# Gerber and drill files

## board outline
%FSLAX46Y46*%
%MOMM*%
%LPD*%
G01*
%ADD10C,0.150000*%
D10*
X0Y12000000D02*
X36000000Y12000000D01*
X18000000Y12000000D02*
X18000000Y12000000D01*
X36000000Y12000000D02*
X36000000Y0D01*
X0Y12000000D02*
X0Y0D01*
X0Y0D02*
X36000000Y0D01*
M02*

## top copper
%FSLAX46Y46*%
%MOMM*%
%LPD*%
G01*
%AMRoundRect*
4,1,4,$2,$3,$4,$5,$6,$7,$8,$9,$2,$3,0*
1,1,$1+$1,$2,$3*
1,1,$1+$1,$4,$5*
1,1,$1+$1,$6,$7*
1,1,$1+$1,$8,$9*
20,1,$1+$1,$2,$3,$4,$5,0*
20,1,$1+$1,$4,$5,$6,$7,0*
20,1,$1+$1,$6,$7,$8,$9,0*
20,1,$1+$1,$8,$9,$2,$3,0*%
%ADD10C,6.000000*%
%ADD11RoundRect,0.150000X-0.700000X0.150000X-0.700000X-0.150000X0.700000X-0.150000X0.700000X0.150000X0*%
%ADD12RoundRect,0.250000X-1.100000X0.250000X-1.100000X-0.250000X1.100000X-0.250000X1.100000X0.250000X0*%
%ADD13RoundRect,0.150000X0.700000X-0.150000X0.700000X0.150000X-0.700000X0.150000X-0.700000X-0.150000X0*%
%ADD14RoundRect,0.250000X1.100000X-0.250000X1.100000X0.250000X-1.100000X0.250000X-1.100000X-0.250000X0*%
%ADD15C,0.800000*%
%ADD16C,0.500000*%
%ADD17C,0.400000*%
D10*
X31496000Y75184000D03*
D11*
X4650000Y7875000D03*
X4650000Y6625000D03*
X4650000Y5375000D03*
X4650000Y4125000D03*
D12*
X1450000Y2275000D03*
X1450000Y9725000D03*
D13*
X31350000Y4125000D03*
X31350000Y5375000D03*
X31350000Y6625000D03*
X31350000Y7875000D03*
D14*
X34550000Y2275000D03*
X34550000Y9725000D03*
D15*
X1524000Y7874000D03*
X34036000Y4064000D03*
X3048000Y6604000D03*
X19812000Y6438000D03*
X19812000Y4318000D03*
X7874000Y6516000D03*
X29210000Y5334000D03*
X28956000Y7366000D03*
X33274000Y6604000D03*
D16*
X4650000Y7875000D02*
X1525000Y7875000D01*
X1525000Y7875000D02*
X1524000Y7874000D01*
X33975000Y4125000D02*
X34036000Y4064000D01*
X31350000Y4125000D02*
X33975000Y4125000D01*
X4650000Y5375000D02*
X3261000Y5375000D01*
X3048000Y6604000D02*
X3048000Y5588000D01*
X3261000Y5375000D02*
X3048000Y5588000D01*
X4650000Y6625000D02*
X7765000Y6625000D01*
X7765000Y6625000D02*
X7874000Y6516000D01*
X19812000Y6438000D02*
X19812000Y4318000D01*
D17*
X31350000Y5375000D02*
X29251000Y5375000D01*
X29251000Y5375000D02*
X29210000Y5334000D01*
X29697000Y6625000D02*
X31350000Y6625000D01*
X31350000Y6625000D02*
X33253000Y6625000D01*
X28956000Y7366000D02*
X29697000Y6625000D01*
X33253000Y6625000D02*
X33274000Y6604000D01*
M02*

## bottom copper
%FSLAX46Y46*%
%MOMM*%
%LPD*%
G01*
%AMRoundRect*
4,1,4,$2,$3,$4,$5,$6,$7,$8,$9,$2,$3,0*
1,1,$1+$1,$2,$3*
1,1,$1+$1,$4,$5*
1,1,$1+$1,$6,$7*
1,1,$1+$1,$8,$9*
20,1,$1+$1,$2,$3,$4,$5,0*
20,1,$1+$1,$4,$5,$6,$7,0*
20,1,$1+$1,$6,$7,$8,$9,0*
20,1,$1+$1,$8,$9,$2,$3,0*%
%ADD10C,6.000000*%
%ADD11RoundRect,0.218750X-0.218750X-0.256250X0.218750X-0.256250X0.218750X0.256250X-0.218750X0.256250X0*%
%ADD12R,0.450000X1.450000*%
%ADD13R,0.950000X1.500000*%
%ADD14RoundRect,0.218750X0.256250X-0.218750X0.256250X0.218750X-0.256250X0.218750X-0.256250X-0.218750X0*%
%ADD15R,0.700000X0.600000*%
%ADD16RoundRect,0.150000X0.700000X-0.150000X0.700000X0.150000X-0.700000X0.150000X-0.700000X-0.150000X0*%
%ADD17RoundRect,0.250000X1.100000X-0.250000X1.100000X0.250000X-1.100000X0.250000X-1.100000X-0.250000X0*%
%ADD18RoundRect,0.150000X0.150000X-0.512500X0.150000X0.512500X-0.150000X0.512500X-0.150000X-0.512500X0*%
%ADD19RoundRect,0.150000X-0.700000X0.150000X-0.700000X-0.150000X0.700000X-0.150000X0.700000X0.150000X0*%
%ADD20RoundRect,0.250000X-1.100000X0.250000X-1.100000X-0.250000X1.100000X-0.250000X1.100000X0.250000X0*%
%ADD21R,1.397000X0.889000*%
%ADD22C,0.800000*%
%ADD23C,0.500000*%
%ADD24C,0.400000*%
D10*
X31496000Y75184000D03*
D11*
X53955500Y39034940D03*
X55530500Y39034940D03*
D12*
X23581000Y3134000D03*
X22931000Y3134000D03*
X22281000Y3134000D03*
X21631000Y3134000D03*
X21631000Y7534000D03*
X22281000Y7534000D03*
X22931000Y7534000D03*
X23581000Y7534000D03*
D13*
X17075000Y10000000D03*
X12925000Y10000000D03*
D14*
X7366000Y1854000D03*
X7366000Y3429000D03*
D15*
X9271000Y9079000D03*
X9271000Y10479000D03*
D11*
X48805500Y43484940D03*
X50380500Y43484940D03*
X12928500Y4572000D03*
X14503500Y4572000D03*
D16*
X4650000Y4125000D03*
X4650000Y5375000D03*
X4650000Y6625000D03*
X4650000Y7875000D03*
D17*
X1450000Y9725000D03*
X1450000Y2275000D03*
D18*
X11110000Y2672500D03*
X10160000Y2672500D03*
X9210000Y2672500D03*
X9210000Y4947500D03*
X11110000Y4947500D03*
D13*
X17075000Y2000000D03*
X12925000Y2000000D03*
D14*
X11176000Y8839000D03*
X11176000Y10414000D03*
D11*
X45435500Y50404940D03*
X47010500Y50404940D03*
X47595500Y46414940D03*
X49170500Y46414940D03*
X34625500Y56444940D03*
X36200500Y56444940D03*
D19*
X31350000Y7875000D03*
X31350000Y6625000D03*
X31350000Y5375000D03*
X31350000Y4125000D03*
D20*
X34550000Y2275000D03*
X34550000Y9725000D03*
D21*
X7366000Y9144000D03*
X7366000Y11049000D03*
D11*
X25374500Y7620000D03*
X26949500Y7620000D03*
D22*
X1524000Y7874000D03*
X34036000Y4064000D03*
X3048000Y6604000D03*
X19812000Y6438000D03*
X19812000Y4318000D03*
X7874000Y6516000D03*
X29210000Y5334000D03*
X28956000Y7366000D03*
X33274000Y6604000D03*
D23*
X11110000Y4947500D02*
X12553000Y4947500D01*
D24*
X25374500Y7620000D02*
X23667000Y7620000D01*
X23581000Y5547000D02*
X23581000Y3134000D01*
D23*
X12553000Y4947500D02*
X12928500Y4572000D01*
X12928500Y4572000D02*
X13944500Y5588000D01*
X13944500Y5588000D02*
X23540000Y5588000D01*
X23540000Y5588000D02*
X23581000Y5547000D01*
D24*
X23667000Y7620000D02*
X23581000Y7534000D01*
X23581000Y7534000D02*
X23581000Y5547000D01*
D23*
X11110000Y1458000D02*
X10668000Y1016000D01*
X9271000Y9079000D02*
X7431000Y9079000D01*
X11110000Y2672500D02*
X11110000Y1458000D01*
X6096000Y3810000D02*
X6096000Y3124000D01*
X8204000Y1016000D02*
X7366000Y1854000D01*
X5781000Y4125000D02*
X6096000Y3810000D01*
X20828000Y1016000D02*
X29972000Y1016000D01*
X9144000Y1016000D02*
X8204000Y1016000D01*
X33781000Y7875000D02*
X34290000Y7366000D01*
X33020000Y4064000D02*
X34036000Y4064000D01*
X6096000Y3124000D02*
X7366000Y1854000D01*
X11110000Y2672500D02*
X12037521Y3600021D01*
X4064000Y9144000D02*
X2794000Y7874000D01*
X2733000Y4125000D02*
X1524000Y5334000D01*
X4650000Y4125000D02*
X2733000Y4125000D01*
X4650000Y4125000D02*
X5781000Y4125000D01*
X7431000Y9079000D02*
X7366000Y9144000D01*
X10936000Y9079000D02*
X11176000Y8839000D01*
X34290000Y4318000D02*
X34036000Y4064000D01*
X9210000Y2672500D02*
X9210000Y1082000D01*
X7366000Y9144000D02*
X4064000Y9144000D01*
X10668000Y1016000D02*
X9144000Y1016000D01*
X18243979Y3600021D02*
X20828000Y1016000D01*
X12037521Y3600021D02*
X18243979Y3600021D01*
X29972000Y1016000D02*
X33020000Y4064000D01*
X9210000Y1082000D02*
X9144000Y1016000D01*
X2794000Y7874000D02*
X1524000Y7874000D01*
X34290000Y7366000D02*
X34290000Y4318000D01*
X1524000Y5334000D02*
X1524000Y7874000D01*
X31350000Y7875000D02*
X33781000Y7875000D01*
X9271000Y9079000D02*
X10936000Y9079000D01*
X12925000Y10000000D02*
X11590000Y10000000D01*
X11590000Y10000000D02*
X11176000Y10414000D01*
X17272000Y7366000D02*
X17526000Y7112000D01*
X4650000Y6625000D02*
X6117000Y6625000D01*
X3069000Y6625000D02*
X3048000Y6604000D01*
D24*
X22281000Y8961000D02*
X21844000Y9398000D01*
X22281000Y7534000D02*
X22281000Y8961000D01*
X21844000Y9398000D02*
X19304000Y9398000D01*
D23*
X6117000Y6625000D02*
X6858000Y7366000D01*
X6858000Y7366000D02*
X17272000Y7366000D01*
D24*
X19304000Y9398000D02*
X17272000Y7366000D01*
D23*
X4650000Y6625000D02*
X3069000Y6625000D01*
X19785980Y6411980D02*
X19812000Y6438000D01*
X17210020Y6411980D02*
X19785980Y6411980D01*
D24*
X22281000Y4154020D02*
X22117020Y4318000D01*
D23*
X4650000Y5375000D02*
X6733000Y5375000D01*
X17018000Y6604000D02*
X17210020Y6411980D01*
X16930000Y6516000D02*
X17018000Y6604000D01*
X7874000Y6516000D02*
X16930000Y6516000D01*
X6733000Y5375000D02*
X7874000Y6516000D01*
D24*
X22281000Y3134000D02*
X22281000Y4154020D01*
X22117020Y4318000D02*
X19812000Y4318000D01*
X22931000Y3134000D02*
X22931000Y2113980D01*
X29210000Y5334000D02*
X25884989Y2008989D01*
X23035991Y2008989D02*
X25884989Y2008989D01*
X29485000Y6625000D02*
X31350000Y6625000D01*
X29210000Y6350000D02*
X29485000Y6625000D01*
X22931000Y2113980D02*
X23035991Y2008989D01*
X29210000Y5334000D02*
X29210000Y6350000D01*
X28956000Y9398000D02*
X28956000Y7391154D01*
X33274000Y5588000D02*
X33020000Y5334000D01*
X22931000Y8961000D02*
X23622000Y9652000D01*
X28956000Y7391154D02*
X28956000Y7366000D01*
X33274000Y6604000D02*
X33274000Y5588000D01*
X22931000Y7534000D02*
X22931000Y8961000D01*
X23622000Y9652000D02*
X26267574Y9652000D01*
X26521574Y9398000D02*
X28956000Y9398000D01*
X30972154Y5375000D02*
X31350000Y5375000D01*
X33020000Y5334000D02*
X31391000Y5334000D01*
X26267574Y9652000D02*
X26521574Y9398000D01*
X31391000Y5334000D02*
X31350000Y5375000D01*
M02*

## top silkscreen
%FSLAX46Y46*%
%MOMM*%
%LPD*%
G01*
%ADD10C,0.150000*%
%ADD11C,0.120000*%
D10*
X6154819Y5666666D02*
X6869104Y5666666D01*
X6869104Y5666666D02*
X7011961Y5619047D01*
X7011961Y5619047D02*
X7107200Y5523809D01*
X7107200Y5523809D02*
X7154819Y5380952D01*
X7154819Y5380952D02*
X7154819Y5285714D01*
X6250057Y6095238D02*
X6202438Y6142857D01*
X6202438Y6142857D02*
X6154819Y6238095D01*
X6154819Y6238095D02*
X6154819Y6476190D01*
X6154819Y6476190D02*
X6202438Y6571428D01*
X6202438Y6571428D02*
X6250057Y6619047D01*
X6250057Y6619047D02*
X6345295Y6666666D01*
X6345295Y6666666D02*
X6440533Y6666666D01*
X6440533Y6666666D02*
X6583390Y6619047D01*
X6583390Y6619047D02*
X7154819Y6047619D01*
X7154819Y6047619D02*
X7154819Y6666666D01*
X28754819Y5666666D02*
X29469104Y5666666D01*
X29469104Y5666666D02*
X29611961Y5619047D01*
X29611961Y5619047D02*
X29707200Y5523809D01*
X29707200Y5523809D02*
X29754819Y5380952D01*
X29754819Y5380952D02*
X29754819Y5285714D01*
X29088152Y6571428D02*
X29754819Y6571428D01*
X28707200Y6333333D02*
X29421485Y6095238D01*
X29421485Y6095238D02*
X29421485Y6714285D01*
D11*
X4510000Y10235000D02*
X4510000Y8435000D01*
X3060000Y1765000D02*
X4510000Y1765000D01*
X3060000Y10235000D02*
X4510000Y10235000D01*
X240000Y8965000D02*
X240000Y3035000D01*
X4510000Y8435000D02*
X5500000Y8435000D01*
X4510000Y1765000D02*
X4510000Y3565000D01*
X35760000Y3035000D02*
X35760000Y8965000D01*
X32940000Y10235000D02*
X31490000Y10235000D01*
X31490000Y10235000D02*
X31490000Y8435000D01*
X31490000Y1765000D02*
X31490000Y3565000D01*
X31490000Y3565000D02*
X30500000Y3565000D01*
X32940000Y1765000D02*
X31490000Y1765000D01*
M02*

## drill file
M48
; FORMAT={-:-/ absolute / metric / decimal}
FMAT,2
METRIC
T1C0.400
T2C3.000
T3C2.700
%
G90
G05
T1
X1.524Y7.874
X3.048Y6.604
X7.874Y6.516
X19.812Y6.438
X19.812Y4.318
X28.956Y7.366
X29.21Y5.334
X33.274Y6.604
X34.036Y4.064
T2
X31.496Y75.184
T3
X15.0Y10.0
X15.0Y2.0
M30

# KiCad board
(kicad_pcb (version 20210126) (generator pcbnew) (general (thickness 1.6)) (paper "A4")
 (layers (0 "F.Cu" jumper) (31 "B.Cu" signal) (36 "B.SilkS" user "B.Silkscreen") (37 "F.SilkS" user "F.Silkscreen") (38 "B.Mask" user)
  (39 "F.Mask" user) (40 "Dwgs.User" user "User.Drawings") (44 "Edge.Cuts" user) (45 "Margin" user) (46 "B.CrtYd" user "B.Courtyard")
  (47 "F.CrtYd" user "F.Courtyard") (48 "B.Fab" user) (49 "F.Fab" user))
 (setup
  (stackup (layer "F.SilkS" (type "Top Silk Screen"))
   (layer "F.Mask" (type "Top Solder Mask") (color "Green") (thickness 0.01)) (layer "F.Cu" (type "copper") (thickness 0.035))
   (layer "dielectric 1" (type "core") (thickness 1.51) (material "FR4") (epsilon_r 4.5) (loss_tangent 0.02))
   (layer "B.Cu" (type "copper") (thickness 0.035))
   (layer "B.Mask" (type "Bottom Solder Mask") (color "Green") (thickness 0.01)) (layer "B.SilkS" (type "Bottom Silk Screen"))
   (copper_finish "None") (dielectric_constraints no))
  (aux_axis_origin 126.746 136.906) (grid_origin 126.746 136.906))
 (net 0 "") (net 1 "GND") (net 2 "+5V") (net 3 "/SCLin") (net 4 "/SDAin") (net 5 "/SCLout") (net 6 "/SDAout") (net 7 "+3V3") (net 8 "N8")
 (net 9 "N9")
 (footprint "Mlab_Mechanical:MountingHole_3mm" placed (layer "F.Cu") (at 31.496 -75.184)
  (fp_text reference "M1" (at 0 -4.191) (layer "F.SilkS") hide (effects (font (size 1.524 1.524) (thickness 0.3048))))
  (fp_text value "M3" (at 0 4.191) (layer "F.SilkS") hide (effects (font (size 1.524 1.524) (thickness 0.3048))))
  (pad "1" thru_hole circle (at 0 0) (locked) (size 6 6) (drill 3) (layers *.Cu *.Adhes *.Mask) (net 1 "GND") (clearance 1) (zone_connect 2)))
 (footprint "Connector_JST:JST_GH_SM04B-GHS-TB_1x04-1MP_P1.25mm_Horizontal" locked (layer "F.Cu") (at 2.8 -6 -90)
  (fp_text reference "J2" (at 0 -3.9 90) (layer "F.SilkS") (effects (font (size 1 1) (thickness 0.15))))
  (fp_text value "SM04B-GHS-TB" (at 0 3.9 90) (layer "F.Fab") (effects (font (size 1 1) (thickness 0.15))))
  (fp_line (start -4.235 -1.71) (end -2.435 -1.71) (layer "F.SilkS") (width 0.12))
  (fp_line (start 4.235 -0.26) (end 4.235 -1.71) (layer "F.SilkS") (width 0.12))
  (fp_line (start -4.235 -0.26) (end -4.235 -1.71) (layer "F.SilkS") (width 0.12))
  (fp_line (start -2.965 2.56) (end 2.965 2.56) (layer "F.SilkS") (width 0.12))
  (fp_line (start -2.435 -1.71) (end -2.435 -2.7) (layer "F.SilkS") (width 0.12))
  (fp_line (start 4.235 -1.71) (end 2.435 -1.71) (layer "F.SilkS") (width 0.12))
  (pad "1" smd roundrect (at -1.875 -1.85 270) (locked) (size 0.6 1.7) (layers "F.Cu" "F.Paste" "F.Mask") (roundrect_rratio 0.25)
   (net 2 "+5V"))
  (pad "2" smd roundrect (at -0.625 -1.85 270) (locked) (size 0.6 1.7) (layers "F.Cu" "F.Paste" "F.Mask") (roundrect_rratio 0.25)
   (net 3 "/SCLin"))
  (pad "3" smd roundrect (at 0.625 -1.85 270) (locked) (size 0.6 1.7) (layers "F.Cu" "F.Paste" "F.Mask") (roundrect_rratio 0.25)
   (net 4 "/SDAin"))
  (pad "4" smd roundrect (at 1.875 -1.85 270) (locked) (size 0.6 1.7) (layers "F.Cu" "F.Paste" "F.Mask") (roundrect_rratio 0.25)
   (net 1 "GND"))
  (pad "MP" smd roundrect (at 3.725 1.35 270) (locked) (size 1 2.7) (layers "F.Cu" "F.Paste" "F.Mask") (roundrect_rratio 0.25) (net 1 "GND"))
  (pad "MP" smd roundrect (at -3.725 1.35 270) (locked) (size 1 2.7) (layers "F.Cu" "F.Paste" "F.Mask") (roundrect_rratio 0.25)
   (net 1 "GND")))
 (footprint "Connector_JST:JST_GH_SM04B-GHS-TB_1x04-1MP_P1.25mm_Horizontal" (layer "F.Cu") (at 33.2 -6 90)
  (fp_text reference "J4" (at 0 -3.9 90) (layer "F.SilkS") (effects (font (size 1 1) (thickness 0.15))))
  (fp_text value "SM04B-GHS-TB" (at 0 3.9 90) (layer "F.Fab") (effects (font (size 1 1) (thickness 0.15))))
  (fp_line (start -2.965 2.56) (end 2.965 2.56) (layer "F.SilkS") (width 0.12))
  (fp_line (start 4.235 -0.26) (end 4.235 -1.71) (layer "F.SilkS") (width 0.12))
  (fp_line (start 4.235 -1.71) (end 2.435 -1.71) (layer "F.SilkS") (width 0.12))
  (fp_line (start -4.235 -1.71) (end -2.435 -1.71) (layer "F.SilkS") (width 0.12))
  (fp_line (start -2.435 -1.71) (end -2.435 -2.7) (layer "F.SilkS") (width 0.12))
  (fp_line (start -4.235 -0.26) (end -4.235 -1.71) (layer "F.SilkS") (width 0.12))
  (pad "1" smd roundrect (at -1.875 -1.85 90) (locked) (size 0.6 1.7) (layers "F.Cu" "F.Paste" "F.Mask") (roundrect_rratio 0.25)
   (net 2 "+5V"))
  (pad "2" smd roundrect (at -0.625 -1.85 90) (locked) (size 0.6 1.7) (layers "F.Cu" "F.Paste" "F.Mask") (roundrect_rratio 0.25)
   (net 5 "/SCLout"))
  (pad "3" smd roundrect (at 0.625 -1.85 90) (locked) (size 0.6 1.7) (layers "F.Cu" "F.Paste" "F.Mask") (roundrect_rratio 0.25)
   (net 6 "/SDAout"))
  (pad "4" smd roundrect (at 1.875 -1.85 90) (locked) (size 0.6 1.7) (layers "F.Cu" "F.Paste" "F.Mask") (roundrect_rratio 0.25)
   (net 1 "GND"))
  (pad "MP" smd roundrect (at -3.725 1.35 90) (locked) (size 1 2.7) (layers "F.Cu" "F.Paste" "F.Mask") (roundrect_rratio 0.25) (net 1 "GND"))
  (pad "MP" smd roundrect (at 3.725 1.35 90) (locked) (size 1 2.7) (layers "F.Cu" "F.Paste" "F.Mask") (roundrect_rratio 0.25) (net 1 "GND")))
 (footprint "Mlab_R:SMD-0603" (layer "B.Cu") (at 54.743 -39.03494)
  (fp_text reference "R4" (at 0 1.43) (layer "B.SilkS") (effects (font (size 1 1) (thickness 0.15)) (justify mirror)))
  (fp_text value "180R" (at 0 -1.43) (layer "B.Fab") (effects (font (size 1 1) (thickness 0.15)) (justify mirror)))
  (pad "1" smd roundrect (at -0.7875 0) (locked) (size 0.875 0.95) (layers "B.Cu" "B.Paste" "B.Mask") (roundrect_rratio 0.25) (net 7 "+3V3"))
  (pad "2" smd roundrect (at 0.7875 0) (locked) (size 0.875 0.95) (layers "B.Cu" "B.Paste" "B.Mask") (roundrect_rratio 0.25) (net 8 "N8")))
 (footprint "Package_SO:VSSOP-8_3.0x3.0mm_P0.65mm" (layer "B.Cu") (at 22.606 -5.334 90)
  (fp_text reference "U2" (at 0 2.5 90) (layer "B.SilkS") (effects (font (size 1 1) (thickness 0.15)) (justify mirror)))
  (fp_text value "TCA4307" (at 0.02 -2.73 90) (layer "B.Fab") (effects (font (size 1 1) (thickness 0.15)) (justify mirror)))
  (pad "1" smd rect (at -2.2 0.975 180) (locked) (size 0.45 1.45) (layers "B.Cu" "B.Paste" "B.Mask") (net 7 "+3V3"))
  (pad "2" smd rect (at -2.2 0.325 180) (locked) (size 0.45 1.45) (layers "B.Cu" "B.Paste" "B.Mask") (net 5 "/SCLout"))
  (pad "3" smd rect (at -2.2 -0.325 180) (locked) (size 0.45 1.45) (layers "B.Cu" "B.Paste" "B.Mask") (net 3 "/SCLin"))
  (pad "4" smd rect (at -2.2 -0.975 180) (locked) (size 0.45 1.45) (layers "B.Cu" "B.Paste" "B.Mask") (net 1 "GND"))
  (pad "5" smd rect (at 2.2 -0.975 180) (locked) (size 0.45 1.45) (layers "B.Cu" "B.Paste" "B.Mask") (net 8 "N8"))
  (pad "6" smd rect (at 2.2 -0.325 180) (locked) (size 0.45 1.45) (layers "B.Cu" "B.Paste" "B.Mask") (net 4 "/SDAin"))
  (pad "7" smd rect (at 2.2 0.325 180) (locked) (size 0.45 1.45) (layers "B.Cu" "B.Paste" "B.Mask") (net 6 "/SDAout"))
  (pad "8" smd rect (at 2.2 0.975 180) (locked) (size 0.45 1.45) (layers "B.Cu" "B.Paste" "B.Mask") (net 7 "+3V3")))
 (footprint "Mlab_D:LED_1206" (layer "B.Cu") (at 15 -10)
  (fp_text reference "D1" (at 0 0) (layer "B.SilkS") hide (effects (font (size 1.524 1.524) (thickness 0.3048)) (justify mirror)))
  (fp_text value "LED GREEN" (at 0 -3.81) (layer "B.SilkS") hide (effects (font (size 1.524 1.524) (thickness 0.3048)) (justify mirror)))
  (pad "" np_thru_hole circle (at 0 0) (locked) (size 2.7 2.7) (drill 2.7) (layers *.Mask))
  (pad "1" smd rect (at 2.075 0) (locked) (size 0.95 1.5) (layers "B.Cu" "B.Paste" "B.Mask") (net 1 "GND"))
  (pad "2" smd rect (at -2.075 0) (locked) (size 0.95 1.5) (layers "B.Cu" "B.Paste" "B.Mask") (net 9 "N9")))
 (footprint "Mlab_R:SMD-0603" (layer "B.Cu") (at 7.366 -2.6415 90)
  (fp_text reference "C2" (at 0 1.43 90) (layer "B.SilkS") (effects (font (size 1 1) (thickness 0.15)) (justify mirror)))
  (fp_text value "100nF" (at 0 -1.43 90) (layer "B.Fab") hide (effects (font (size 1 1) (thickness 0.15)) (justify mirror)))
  (pad "1" smd roundrect (at -0.7875 0 90) (locked) (size 0.875 0.95) (layers "B.Cu" "B.Paste" "B.Mask") (roundrect_rratio 0.25)
   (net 2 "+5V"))
  (pad "2" smd roundrect (at 0.7875 0 90) (locked) (size 0.875 0.95) (layers "B.Cu" "B.Paste" "B.Mask") (roundrect_rratio 0.25)
   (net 1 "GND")))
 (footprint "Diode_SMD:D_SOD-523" (layer "B.Cu") (at 9.271 -9.779 90)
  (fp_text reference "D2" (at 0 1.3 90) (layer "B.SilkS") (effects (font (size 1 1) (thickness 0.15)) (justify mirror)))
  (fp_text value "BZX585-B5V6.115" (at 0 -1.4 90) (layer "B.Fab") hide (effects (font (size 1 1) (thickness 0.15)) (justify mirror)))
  (pad "1" smd rect (at -0.7 0 270) (locked) (size 0.6 0.7) (layers "B.Cu" "B.Paste" "B.Mask") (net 2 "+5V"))
  (pad "2" smd rect (at 0.7 0 270) (locked) (size 0.6 0.7) (layers "B.Cu" "B.Paste" "B.Mask") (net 1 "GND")))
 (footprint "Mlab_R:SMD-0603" (layer "B.Cu") (at 49.593 -43.48494)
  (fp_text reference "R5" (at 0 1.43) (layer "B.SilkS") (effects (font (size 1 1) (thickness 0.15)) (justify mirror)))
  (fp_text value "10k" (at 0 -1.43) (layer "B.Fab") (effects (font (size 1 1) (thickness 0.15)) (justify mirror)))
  (pad "1" smd roundrect (at -0.7875 0) (locked) (size 0.875 0.95) (layers "B.Cu" "B.Paste" "B.Mask") (roundrect_rratio 0.25) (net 7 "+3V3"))
  (pad "2" smd roundrect (at 0.7875 0) (locked) (size 0.875 0.95) (layers "B.Cu" "B.Paste" "B.Mask") (roundrect_rratio 0.25)
   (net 5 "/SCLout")))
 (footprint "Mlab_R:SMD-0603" (layer "B.Cu") (at 13.716 -4.572)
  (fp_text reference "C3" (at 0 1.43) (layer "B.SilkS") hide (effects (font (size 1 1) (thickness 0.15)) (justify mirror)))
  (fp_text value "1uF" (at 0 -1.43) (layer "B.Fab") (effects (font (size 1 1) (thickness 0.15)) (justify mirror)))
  (pad "1" smd roundrect (at -0.7875 0) (locked) (size 0.875 0.95) (layers "B.Cu" "B.Paste" "B.Mask") (roundrect_rratio 0.25) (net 7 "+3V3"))
  (pad "2" smd roundrect (at 0.7875 0) (locked) (size 0.875 0.95) (layers "B.Cu" "B.Paste" "B.Mask") (roundrect_rratio 0.25) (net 1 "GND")))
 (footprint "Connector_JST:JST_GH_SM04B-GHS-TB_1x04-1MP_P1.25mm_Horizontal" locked (layer "B.Cu") (at 2.8 -6 90)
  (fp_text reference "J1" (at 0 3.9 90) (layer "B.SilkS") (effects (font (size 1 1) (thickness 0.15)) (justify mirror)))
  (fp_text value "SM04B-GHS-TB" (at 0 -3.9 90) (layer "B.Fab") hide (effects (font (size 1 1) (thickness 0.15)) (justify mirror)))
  (pad "1" smd roundrect (at -1.875 1.85 90) (locked) (size 0.6 1.7) (layers "B.Cu" "B.Paste" "B.Mask") (roundrect_rratio 0.25)
   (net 2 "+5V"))
  (pad "2" smd roundrect (at -0.625 1.85 90) (locked) (size 0.6 1.7) (layers "B.Cu" "B.Paste" "B.Mask") (roundrect_rratio 0.25)
   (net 3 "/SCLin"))
  (pad "3" smd roundrect (at 0.625 1.85 90) (locked) (size 0.6 1.7) (layers "B.Cu" "B.Paste" "B.Mask") (roundrect_rratio 0.25)
   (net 4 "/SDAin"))
  (pad "4" smd roundrect (at 1.875 1.85 90) (locked) (size 0.6 1.7) (layers "B.Cu" "B.Paste" "B.Mask") (roundrect_rratio 0.25) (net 1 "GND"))
  (pad "MP" smd roundrect (at 3.725 -1.35 90) (locked) (size 1 2.7) (layers "B.Cu" "B.Paste" "B.Mask") (roundrect_rratio 0.25) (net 1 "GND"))
  (pad "MP" smd roundrect (at -3.725 -1.35 90) (locked) (size 1 2.7) (layers "B.Cu" "B.Paste" "B.Mask") (roundrect_rratio 0.25)
   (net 1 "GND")))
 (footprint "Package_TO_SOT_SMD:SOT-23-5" (layer "B.Cu") (at 10.16 -3.81 90)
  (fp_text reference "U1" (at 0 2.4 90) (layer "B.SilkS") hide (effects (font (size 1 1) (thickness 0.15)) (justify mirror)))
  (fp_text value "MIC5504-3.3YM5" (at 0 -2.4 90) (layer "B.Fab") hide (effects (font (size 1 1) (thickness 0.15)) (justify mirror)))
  (pad "1" smd roundrect (at -1.1375 0.95 90) (locked) (size 1.325 0.6) (layers "B.Cu" "B.Paste" "B.Mask") (roundrect_rratio 0.25)
   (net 2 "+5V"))
  (pad "2" smd roundrect (at -1.1375 0 90) (locked) (size 1.325 0.6) (layers "B.Cu" "B.Paste" "B.Mask") (roundrect_rratio 0.25)
   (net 1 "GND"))
  (pad "3" smd roundrect (at -1.1375 -0.95 90) (locked) (size 1.325 0.6) (layers "B.Cu" "B.Paste" "B.Mask") (roundrect_rratio 0.25)
   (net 2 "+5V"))
  (pad "4" smd roundrect (at 1.1375 -0.95 90) (locked) (size 1.325 0.6) (layers "B.Cu" "B.Paste" "B.Mask") (roundrect_rratio 0.25))
  (pad "5" smd roundrect (at 1.1375 0.95 90) (locked) (size 1.325 0.6) (layers "B.Cu" "B.Paste" "B.Mask") (roundrect_rratio 0.25)
   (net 7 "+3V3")))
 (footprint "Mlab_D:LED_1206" (layer "B.Cu") (at 15 -2)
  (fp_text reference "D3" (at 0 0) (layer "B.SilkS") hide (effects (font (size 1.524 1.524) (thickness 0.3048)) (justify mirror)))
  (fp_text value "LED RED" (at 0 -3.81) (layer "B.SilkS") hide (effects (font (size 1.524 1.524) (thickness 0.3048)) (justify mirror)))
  (pad "" np_thru_hole circle (at 0 0) (locked) (size 2.7 2.7) (drill 2.7) (layers *.Mask))
  (pad "1" smd rect (at 2.075 0) (locked) (size 0.95 1.5) (layers "B.Cu" "B.Paste" "B.Mask") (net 1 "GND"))
  (pad "2" smd rect (at -2.075 0) (locked) (size 0.95 1.5) (layers "B.Cu" "B.Paste" "B.Mask") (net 8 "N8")))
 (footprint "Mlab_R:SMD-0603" (layer "B.Cu") (at 11.176 -9.6265 90)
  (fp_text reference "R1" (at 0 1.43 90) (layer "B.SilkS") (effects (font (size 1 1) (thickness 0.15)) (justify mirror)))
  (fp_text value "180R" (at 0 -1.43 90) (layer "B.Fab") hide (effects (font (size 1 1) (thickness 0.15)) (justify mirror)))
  (pad "1" smd roundrect (at -0.7875 0 90) (locked) (size 0.875 0.95) (layers "B.Cu" "B.Paste" "B.Mask") (roundrect_rratio 0.25)
   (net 2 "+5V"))
  (pad "2" smd roundrect (at 0.7875 0 90) (locked) (size 0.875 0.95) (layers "B.Cu" "B.Paste" "B.Mask") (roundrect_rratio 0.25) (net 9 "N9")))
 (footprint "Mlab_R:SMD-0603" (layer "B.Cu") (at 46.223 -50.40494)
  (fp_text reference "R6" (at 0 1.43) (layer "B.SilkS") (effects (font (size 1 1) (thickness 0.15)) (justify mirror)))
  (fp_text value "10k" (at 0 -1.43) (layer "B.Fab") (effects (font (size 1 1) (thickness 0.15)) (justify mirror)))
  (pad "1" smd roundrect (at -0.7875 0) (locked) (size 0.875 0.95) (layers "B.Cu" "B.Paste" "B.Mask") (roundrect_rratio 0.25) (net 7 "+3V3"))
  (pad "2" smd roundrect (at 0.7875 0) (locked) (size 0.875 0.95) (layers "B.Cu" "B.Paste" "B.Mask") (roundrect_rratio 0.25)
   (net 6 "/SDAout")))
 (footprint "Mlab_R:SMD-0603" (layer "B.Cu") (at 48.383 -46.41494)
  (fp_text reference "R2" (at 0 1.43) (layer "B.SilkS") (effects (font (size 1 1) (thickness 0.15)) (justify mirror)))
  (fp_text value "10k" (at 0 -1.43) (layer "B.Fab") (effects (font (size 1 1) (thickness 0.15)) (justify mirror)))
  (pad "1" smd roundrect (at -0.7875 0) (locked) (size 0.875 0.95) (layers "B.Cu" "B.Paste" "B.Mask") (roundrect_rratio 0.25) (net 7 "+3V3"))
  (pad "2" smd roundrect (at 0.7875 0) (locked) (size 0.875 0.95) (layers "B.Cu" "B.Paste" "B.Mask") (roundrect_rratio 0.25)
   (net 3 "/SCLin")))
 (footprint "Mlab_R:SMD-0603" (layer "B.Cu") (at 35.413 -56.44494)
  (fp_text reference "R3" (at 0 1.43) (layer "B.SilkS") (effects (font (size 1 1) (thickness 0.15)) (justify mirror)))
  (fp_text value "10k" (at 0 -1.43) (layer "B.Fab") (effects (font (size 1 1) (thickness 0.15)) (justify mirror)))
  (pad "1" smd roundrect (at -0.7875 0) (locked) (size 0.875 0.95) (layers "B.Cu" "B.Paste" "B.Mask") (roundrect_rratio 0.25) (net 7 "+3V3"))
  (pad "2" smd roundrect (at 0.7875 0) (locked) (size 0.875 0.95) (layers "B.Cu" "B.Paste" "B.Mask") (roundrect_rratio 0.25)
   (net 4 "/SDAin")))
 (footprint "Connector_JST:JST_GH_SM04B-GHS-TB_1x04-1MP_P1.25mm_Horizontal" (layer "B.Cu") (at 33.2 -6 -90)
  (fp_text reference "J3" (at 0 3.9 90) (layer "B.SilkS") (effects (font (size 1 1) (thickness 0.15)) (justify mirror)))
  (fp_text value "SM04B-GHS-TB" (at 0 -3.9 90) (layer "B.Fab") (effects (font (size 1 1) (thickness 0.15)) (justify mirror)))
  (pad "1" smd roundrect (at -1.875 1.85 270) (locked) (size 0.6 1.7) (layers "B.Cu" "B.Paste" "B.Mask") (roundrect_rratio 0.25)
   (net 2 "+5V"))
  (pad "2" smd roundrect (at -0.625 1.85 270) (locked) (size 0.6 1.7) (layers "B.Cu" "B.Paste" "B.Mask") (roundrect_rratio 0.25)
   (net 5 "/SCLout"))
  (pad "3" smd roundrect (at 0.625 1.85 270) (locked) (size 0.6 1.7) (layers "B.Cu" "B.Paste" "B.Mask") (roundrect_rratio 0.25)
   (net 6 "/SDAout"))
  (pad "4" smd roundrect (at 1.875 1.85 270) (locked) (size 0.6 1.7) (layers "B.Cu" "B.Paste" "B.Mask") (roundrect_rratio 0.25)
   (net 1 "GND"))
  (pad "MP" smd roundrect (at 3.725 -1.35 270) (locked) (size 1 2.7) (layers "B.Cu" "B.Paste" "B.Mask") (roundrect_rratio 0.25)
   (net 1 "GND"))
  (pad "MP" smd roundrect (at -3.725 -1.35 270) (locked) (size 1 2.7) (layers "B.Cu" "B.Paste" "B.Mask") (roundrect_rratio 0.25)
   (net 1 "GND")))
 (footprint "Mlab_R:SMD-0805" (layer "B.Cu") (at 7.366 -10.0965 90)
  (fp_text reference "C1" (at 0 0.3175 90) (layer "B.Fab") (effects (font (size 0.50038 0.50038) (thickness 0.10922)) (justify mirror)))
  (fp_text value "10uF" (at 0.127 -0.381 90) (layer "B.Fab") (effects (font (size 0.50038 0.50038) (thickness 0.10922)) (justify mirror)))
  (pad "1" smd rect (at -0.9525 0 90) (locked) (size 0.889 1.397) (layers "B.Cu" "B.Paste" "B.Mask") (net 2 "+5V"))
  (pad "2" smd rect (at 0.9525 0 90) (locked) (size 0.889 1.397) (layers "B.Cu" "B.Paste" "B.Mask") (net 1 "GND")))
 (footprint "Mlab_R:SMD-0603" (layer "B.Cu") (at 26.162 -7.62)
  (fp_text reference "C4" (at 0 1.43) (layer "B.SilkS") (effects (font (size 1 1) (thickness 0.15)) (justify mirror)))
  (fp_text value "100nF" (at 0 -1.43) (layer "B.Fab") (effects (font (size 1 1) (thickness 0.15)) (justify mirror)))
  (pad "1" smd roundrect (at -0.7875 0) (locked) (size 0.875 0.95) (layers "B.Cu" "B.Paste" "B.Mask") (roundrect_rratio 0.25) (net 7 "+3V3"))
  (pad "2" smd roundrect (at 0.7875 0) (locked) (size 0.875 0.95) (layers "B.Cu" "B.Paste" "B.Mask") (roundrect_rratio 0.25) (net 1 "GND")))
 (gr_line (start 0 -12) (end 36 -12) (layer "Edge.Cuts") (width 0.15))
 (gr_line (start 18 -12) (end 18 -12) (layer "Edge.Cuts") (width 0.15) (locked))
 (gr_line (start 36 -12) (end 36 0) (layer "Edge.Cuts") (width 0.15) (locked))
 (gr_line (start 0 -12) (end 0 0) (layer "Edge.Cuts") (width 0.15) (locked))
 (gr_line (start 0 0) (end 36 0) (layer "Edge.Cuts") (width 0.15) (locked))
 (segment (start 11.11 -4.9475) (end 12.553 -4.9475) (width 0.5) (layer "B.Cu") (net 7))
 (segment (start 25.3745 -7.62) (end 23.667 -7.62) (width 0.4) (layer "B.Cu") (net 7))
 (segment (start 23.581 -5.547) (end 23.581 -3.134) (width 0.4) (layer "B.Cu") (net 7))
 (segment (start 12.553 -4.9475) (end 12.9285 -4.572) (width 0.5) (layer "B.Cu") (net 7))
 (segment (start 12.9285 -4.572) (end 13.9445 -5.588) (width 0.5) (layer "B.Cu") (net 7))
 (segment (start 13.9445 -5.588) (end 23.54 -5.588) (width 0.5) (layer "B.Cu") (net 7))
 (segment (start 23.54 -5.588) (end 23.581 -5.547) (width 0.5) (layer "B.Cu") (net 7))
 (segment (start 23.667 -7.62) (end 23.581 -7.534) (width 0.4) (layer "B.Cu") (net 7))
 (segment (start 23.581 -7.534) (end 23.581 -5.547) (width 0.4) (layer "B.Cu") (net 7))
 (segment (start 4.65 -7.875) (end 1.525 -7.875) (width 0.5) (layer "F.Cu") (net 2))
 (segment (start 1.525 -7.875) (end 1.524 -7.874) (width 0.5) (layer "F.Cu") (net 2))
 (segment (start 33.975 -4.125) (end 34.036 -4.064) (width 0.5) (layer "F.Cu") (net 2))
 (segment (start 31.35 -4.125) (end 33.975 -4.125) (width 0.5) (layer "F.Cu") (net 2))
 (via (at 1.524 -7.874) (size 0.8) (drill 0.4) (layers "F.Cu" "B.Cu") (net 2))
 (via (at 34.036 -4.064) (size 0.8) (drill 0.4) (layers "F.Cu" "B.Cu") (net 2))
 (segment (start 11.11 -1.458) (end 10.668 -1.016) (width 0.5) (layer "B.Cu") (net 2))
 (segment (start 9.271 -9.079) (end 7.431 -9.079) (width 0.5) (layer "B.Cu") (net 2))
 (segment (start 11.11 -2.6725) (end 11.11 -1.458) (width 0.5) (layer "B.Cu") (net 2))
 (segment (start 6.096 -3.81) (end 6.096 -3.124) (width 0.5) (layer "B.Cu") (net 2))
 (segment (start 8.204 -1.016) (end 7.366 -1.854) (width 0.5) (layer "B.Cu") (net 2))
 (segment (start 5.781 -4.125) (end 6.096 -3.81) (width 0.5) (layer "B.Cu") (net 2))
 (segment (start 20.828 -1.016) (end 29.972 -1.016) (width 0.5) (layer "B.Cu") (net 2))
 (segment (start 9.144 -1.016) (end 8.204 -1.016) (width 0.5) (layer "B.Cu") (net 2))
 (segment (start 33.781 -7.875) (end 34.29 -7.366) (width 0.5) (layer "B.Cu") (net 2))
 (segment (start 33.02 -4.064) (end 34.036 -4.064) (width 0.5) (layer "B.Cu") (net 2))
 (segment (start 6.096 -3.124) (end 7.366 -1.854) (width 0.5) (layer "B.Cu") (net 2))
 (segment (start 11.11 -2.6725) (end 12.037521 -3.600021) (width 0.5) (layer "B.Cu") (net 2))
 (segment (start 4.064 -9.144) (end 2.794 -7.874) (width 0.5) (layer "B.Cu") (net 2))
 (segment (start 2.733 -4.125) (end 1.524 -5.334) (width 0.5) (layer "B.Cu") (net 2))
 (segment (start 4.65 -4.125) (end 2.733 -4.125) (width 0.5) (layer "B.Cu") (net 2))
 (segment (start 4.65 -4.125) (end 5.781 -4.125) (width 0.5) (layer "B.Cu") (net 2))
 (segment (start 7.431 -9.079) (end 7.366 -9.144) (width 0.5) (layer "B.Cu") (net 2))
 (segment (start 10.936 -9.079) (end 11.176 -8.839) (width 0.5) (layer "B.Cu") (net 2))
 (segment (start 34.29 -4.318) (end 34.036 -4.064) (width 0.5) (layer "B.Cu") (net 2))
 (segment (start 9.21 -2.6725) (end 9.21 -1.082) (width 0.5) (layer "B.Cu") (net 2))
 (segment (start 7.366 -9.144) (end 4.064 -9.144) (width 0.5) (layer "B.Cu") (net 2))
 (segment (start 10.668 -1.016) (end 9.144 -1.016) (width 0.5) (layer "B.Cu") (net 2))
 (segment (start 18.243979 -3.600021) (end 20.828 -1.016) (width 0.5) (layer "B.Cu") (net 2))
 (segment (start 12.037521 -3.600021) (end 18.243979 -3.600021) (width 0.5) (layer "B.Cu") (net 2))
 (segment (start 29.972 -1.016) (end 33.02 -4.064) (width 0.5) (layer "B.Cu") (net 2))
 (segment (start 9.21 -1.082) (end 9.144 -1.016) (width 0.5) (layer "B.Cu") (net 2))
 (segment (start 2.794 -7.874) (end 1.524 -7.874) (width 0.5) (layer "B.Cu") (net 2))
 (segment (start 34.29 -7.366) (end 34.29 -4.318) (width 0.5) (layer "B.Cu") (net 2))
 (segment (start 1.524 -5.334) (end 1.524 -7.874) (width 0.5) (layer "B.Cu") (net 2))
 (segment (start 31.35 -7.875) (end 33.781 -7.875) (width 0.5) (layer "B.Cu") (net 2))
 (segment (start 9.271 -9.079) (end 10.936 -9.079) (width 0.5) (layer "B.Cu") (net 2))
 (segment (start 12.925 -10) (end 11.59 -10) (width 0.5) (layer "B.Cu") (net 9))
 (segment (start 11.59 -10) (end 11.176 -10.414) (width 0.5) (layer "B.Cu") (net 9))
 (segment (start 4.65 -5.375) (end 3.261 -5.375) (width 0.5) (layer "F.Cu") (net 4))
 (segment (start 3.048 -6.604) (end 3.048 -5.588) (width 0.5) (layer "F.Cu") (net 4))
 (segment (start 3.261 -5.375) (end 3.048 -5.588) (width 0.5) (layer "F.Cu") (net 4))
 (via (at 3.048 -6.604) (size 0.8) (drill 0.4) (layers "F.Cu" "B.Cu") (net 4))
 (segment (start 17.272 -7.366) (end 17.526 -7.112) (width 0.5) (layer "B.Cu") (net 4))
 (segment (start 4.65 -6.625) (end 6.117 -6.625) (width 0.5) (layer "B.Cu") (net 4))
 (segment (start 3.069 -6.625) (end 3.048 -6.604) (width 0.5) (layer "B.Cu") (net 4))
 (segment (start 22.281 -8.961) (end 21.844 -9.398) (width 0.4) (layer "B.Cu") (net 4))
 (segment (start 22.281 -7.534) (end 22.281 -8.961) (width 0.4) (layer "B.Cu") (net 4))
 (segment (start 21.844 -9.398) (end 19.304 -9.398) (width 0.4) (layer "B.Cu") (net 4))
 (segment (start 6.117 -6.625) (end 6.858 -7.366) (width 0.5) (layer "B.Cu") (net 4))
 (segment (start 6.858 -7.366) (end 17.272 -7.366) (width 0.5) (layer "B.Cu") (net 4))
 (segment (start 19.304 -9.398) (end 17.272 -7.366) (width 0.4) (layer "B.Cu") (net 4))
 (segment (start 4.65 -6.625) (end 3.069 -6.625) (width 0.5) (layer "B.Cu") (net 4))
 (segment (start 4.65 -6.625) (end 7.765 -6.625) (width 0.5) (layer "F.Cu") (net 3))
 (segment (start 7.765 -6.625) (end 7.874 -6.516) (width 0.5) (layer "F.Cu") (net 3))
 (segment (start 19.812 -6.438) (end 19.812 -4.318) (width 0.5) (layer "F.Cu") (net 3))
 (via (at 19.812 -6.438) (size 0.8) (drill 0.4) (layers "F.Cu" "B.Cu") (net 3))
 (via (at 19.812 -4.318) (size 0.8) (drill 0.4) (layers "F.Cu" "B.Cu") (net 3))
 (via (at 7.874 -6.516) (size 0.8) (drill 0.4) (layers "F.Cu" "B.Cu") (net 3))
 (segment (start 19.78598 -6.41198) (end 19.812 -6.438) (width 0.5) (layer "B.Cu") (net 3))
 (segment (start 17.21002 -6.41198) (end 19.78598 -6.41198) (width 0.5) (layer "B.Cu") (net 3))
 (segment (start 22.281 -4.15402) (end 22.11702 -4.318) (width 0.4) (layer "B.Cu") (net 3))
 (segment (start 4.65 -5.375) (end 6.733 -5.375) (width 0.5) (layer "B.Cu") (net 3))
 (segment (start 17.018 -6.604) (end 17.21002 -6.41198) (width 0.5) (layer "B.Cu") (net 3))
 (segment (start 16.93 -6.516) (end 17.018 -6.604) (width 0.5) (layer "B.Cu") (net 3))
 (segment (start 7.874 -6.516) (end 16.93 -6.516) (width 0.5) (layer "B.Cu") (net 3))
 (segment (start 6.733 -5.375) (end 7.874 -6.516) (width 0.5) (layer "B.Cu") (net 3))
 (segment (start 22.281 -3.134) (end 22.281 -4.15402) (width 0.4) (layer "B.Cu") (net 3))
 (segment (start 22.11702 -4.318) (end 19.812 -4.318) (width 0.4) (layer "B.Cu") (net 3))
 (segment (start 31.35 -5.375) (end 29.251 -5.375) (width 0.4) (layer "F.Cu") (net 5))
 (segment (start 29.251 -5.375) (end 29.21 -5.334) (width 0.4) (layer "F.Cu") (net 5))
 (via (at 29.21 -5.334) (size 0.8) (drill 0.4) (layers "F.Cu" "B.Cu") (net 5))
 (segment (start 22.931 -3.134) (end 22.931 -2.11398) (width 0.4) (layer "B.Cu") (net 5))
 (segment (start 29.21 -5.334) (end 25.884989 -2.008989) (width 0.4) (layer "B.Cu") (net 5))
 (segment (start 23.035991 -2.008989) (end 25.884989 -2.008989) (width 0.4) (layer "B.Cu") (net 5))
 (segment (start 29.485 -6.625) (end 31.35 -6.625) (width 0.4) (layer "B.Cu") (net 5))
 (segment (start 29.21 -6.35) (end 29.485 -6.625) (width 0.4) (layer "B.Cu") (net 5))
 (segment (start 22.931 -2.11398) (end 23.035991 -2.008989) (width 0.4) (layer "B.Cu") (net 5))
 (segment (start 29.21 -5.334) (end 29.21 -6.35) (width 0.4) (layer "B.Cu") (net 5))
 (segment (start 29.697 -6.625) (end 31.35 -6.625) (width 0.4) (layer "F.Cu") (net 6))
 (segment (start 31.35 -6.625) (end 33.253 -6.625) (width 0.4) (layer "F.Cu") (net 6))
 (segment (start 28.956 -7.366) (end 29.697 -6.625) (width 0.4) (layer "F.Cu") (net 6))
 (segment (start 33.253 -6.625) (end 33.274 -6.604) (width 0.4) (layer "F.Cu") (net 6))
 (via (at 28.956 -7.366) (size 0.8) (drill 0.4) (layers "F.Cu" "B.Cu") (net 6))
 (via (at 33.274 -6.604) (size 0.8) (drill 0.4) (layers "F.Cu" "B.Cu") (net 6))
 (segment (start 28.956 -9.398) (end 28.956 -7.391154) (width 0.4) (layer "B.Cu") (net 6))
 (segment (start 33.274 -5.588) (end 33.02 -5.334) (width 0.4) (layer "B.Cu") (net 6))
 (segment (start 22.931 -8.961) (end 23.622 -9.652) (width 0.4) (layer "B.Cu") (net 6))
 (segment (start 28.956 -7.391154) (end 28.956 -7.366) (width 0.4) (layer "B.Cu") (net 6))
 (segment (start 33.274 -6.604) (end 33.274 -5.588) (width 0.4) (layer "B.Cu") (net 6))
 (segment (start 22.931 -7.534) (end 22.931 -8.961) (width 0.4) (layer "B.Cu") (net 6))
 (segment (start 23.622 -9.652) (end 26.267574 -9.652) (width 0.4) (layer "B.Cu") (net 6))
 (segment (start 26.521574 -9.398) (end 28.956 -9.398) (width 0.4) (layer "B.Cu") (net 6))
 (segment (start 30.972154 -5.375) (end 31.35 -5.375) (width 0.4) (layer "B.Cu") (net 6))
 (segment (start 33.02 -5.334) (end 31.391 -5.334) (width 0.4) (layer "B.Cu") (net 6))
 (segment (start 26.267574 -9.652) (end 26.521574 -9.398) (width 0.4) (layer "B.Cu") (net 6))
 (segment (start 31.391 -5.334) (end 31.35 -5.375) (width 0.4) (layer "B.Cu") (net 6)))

